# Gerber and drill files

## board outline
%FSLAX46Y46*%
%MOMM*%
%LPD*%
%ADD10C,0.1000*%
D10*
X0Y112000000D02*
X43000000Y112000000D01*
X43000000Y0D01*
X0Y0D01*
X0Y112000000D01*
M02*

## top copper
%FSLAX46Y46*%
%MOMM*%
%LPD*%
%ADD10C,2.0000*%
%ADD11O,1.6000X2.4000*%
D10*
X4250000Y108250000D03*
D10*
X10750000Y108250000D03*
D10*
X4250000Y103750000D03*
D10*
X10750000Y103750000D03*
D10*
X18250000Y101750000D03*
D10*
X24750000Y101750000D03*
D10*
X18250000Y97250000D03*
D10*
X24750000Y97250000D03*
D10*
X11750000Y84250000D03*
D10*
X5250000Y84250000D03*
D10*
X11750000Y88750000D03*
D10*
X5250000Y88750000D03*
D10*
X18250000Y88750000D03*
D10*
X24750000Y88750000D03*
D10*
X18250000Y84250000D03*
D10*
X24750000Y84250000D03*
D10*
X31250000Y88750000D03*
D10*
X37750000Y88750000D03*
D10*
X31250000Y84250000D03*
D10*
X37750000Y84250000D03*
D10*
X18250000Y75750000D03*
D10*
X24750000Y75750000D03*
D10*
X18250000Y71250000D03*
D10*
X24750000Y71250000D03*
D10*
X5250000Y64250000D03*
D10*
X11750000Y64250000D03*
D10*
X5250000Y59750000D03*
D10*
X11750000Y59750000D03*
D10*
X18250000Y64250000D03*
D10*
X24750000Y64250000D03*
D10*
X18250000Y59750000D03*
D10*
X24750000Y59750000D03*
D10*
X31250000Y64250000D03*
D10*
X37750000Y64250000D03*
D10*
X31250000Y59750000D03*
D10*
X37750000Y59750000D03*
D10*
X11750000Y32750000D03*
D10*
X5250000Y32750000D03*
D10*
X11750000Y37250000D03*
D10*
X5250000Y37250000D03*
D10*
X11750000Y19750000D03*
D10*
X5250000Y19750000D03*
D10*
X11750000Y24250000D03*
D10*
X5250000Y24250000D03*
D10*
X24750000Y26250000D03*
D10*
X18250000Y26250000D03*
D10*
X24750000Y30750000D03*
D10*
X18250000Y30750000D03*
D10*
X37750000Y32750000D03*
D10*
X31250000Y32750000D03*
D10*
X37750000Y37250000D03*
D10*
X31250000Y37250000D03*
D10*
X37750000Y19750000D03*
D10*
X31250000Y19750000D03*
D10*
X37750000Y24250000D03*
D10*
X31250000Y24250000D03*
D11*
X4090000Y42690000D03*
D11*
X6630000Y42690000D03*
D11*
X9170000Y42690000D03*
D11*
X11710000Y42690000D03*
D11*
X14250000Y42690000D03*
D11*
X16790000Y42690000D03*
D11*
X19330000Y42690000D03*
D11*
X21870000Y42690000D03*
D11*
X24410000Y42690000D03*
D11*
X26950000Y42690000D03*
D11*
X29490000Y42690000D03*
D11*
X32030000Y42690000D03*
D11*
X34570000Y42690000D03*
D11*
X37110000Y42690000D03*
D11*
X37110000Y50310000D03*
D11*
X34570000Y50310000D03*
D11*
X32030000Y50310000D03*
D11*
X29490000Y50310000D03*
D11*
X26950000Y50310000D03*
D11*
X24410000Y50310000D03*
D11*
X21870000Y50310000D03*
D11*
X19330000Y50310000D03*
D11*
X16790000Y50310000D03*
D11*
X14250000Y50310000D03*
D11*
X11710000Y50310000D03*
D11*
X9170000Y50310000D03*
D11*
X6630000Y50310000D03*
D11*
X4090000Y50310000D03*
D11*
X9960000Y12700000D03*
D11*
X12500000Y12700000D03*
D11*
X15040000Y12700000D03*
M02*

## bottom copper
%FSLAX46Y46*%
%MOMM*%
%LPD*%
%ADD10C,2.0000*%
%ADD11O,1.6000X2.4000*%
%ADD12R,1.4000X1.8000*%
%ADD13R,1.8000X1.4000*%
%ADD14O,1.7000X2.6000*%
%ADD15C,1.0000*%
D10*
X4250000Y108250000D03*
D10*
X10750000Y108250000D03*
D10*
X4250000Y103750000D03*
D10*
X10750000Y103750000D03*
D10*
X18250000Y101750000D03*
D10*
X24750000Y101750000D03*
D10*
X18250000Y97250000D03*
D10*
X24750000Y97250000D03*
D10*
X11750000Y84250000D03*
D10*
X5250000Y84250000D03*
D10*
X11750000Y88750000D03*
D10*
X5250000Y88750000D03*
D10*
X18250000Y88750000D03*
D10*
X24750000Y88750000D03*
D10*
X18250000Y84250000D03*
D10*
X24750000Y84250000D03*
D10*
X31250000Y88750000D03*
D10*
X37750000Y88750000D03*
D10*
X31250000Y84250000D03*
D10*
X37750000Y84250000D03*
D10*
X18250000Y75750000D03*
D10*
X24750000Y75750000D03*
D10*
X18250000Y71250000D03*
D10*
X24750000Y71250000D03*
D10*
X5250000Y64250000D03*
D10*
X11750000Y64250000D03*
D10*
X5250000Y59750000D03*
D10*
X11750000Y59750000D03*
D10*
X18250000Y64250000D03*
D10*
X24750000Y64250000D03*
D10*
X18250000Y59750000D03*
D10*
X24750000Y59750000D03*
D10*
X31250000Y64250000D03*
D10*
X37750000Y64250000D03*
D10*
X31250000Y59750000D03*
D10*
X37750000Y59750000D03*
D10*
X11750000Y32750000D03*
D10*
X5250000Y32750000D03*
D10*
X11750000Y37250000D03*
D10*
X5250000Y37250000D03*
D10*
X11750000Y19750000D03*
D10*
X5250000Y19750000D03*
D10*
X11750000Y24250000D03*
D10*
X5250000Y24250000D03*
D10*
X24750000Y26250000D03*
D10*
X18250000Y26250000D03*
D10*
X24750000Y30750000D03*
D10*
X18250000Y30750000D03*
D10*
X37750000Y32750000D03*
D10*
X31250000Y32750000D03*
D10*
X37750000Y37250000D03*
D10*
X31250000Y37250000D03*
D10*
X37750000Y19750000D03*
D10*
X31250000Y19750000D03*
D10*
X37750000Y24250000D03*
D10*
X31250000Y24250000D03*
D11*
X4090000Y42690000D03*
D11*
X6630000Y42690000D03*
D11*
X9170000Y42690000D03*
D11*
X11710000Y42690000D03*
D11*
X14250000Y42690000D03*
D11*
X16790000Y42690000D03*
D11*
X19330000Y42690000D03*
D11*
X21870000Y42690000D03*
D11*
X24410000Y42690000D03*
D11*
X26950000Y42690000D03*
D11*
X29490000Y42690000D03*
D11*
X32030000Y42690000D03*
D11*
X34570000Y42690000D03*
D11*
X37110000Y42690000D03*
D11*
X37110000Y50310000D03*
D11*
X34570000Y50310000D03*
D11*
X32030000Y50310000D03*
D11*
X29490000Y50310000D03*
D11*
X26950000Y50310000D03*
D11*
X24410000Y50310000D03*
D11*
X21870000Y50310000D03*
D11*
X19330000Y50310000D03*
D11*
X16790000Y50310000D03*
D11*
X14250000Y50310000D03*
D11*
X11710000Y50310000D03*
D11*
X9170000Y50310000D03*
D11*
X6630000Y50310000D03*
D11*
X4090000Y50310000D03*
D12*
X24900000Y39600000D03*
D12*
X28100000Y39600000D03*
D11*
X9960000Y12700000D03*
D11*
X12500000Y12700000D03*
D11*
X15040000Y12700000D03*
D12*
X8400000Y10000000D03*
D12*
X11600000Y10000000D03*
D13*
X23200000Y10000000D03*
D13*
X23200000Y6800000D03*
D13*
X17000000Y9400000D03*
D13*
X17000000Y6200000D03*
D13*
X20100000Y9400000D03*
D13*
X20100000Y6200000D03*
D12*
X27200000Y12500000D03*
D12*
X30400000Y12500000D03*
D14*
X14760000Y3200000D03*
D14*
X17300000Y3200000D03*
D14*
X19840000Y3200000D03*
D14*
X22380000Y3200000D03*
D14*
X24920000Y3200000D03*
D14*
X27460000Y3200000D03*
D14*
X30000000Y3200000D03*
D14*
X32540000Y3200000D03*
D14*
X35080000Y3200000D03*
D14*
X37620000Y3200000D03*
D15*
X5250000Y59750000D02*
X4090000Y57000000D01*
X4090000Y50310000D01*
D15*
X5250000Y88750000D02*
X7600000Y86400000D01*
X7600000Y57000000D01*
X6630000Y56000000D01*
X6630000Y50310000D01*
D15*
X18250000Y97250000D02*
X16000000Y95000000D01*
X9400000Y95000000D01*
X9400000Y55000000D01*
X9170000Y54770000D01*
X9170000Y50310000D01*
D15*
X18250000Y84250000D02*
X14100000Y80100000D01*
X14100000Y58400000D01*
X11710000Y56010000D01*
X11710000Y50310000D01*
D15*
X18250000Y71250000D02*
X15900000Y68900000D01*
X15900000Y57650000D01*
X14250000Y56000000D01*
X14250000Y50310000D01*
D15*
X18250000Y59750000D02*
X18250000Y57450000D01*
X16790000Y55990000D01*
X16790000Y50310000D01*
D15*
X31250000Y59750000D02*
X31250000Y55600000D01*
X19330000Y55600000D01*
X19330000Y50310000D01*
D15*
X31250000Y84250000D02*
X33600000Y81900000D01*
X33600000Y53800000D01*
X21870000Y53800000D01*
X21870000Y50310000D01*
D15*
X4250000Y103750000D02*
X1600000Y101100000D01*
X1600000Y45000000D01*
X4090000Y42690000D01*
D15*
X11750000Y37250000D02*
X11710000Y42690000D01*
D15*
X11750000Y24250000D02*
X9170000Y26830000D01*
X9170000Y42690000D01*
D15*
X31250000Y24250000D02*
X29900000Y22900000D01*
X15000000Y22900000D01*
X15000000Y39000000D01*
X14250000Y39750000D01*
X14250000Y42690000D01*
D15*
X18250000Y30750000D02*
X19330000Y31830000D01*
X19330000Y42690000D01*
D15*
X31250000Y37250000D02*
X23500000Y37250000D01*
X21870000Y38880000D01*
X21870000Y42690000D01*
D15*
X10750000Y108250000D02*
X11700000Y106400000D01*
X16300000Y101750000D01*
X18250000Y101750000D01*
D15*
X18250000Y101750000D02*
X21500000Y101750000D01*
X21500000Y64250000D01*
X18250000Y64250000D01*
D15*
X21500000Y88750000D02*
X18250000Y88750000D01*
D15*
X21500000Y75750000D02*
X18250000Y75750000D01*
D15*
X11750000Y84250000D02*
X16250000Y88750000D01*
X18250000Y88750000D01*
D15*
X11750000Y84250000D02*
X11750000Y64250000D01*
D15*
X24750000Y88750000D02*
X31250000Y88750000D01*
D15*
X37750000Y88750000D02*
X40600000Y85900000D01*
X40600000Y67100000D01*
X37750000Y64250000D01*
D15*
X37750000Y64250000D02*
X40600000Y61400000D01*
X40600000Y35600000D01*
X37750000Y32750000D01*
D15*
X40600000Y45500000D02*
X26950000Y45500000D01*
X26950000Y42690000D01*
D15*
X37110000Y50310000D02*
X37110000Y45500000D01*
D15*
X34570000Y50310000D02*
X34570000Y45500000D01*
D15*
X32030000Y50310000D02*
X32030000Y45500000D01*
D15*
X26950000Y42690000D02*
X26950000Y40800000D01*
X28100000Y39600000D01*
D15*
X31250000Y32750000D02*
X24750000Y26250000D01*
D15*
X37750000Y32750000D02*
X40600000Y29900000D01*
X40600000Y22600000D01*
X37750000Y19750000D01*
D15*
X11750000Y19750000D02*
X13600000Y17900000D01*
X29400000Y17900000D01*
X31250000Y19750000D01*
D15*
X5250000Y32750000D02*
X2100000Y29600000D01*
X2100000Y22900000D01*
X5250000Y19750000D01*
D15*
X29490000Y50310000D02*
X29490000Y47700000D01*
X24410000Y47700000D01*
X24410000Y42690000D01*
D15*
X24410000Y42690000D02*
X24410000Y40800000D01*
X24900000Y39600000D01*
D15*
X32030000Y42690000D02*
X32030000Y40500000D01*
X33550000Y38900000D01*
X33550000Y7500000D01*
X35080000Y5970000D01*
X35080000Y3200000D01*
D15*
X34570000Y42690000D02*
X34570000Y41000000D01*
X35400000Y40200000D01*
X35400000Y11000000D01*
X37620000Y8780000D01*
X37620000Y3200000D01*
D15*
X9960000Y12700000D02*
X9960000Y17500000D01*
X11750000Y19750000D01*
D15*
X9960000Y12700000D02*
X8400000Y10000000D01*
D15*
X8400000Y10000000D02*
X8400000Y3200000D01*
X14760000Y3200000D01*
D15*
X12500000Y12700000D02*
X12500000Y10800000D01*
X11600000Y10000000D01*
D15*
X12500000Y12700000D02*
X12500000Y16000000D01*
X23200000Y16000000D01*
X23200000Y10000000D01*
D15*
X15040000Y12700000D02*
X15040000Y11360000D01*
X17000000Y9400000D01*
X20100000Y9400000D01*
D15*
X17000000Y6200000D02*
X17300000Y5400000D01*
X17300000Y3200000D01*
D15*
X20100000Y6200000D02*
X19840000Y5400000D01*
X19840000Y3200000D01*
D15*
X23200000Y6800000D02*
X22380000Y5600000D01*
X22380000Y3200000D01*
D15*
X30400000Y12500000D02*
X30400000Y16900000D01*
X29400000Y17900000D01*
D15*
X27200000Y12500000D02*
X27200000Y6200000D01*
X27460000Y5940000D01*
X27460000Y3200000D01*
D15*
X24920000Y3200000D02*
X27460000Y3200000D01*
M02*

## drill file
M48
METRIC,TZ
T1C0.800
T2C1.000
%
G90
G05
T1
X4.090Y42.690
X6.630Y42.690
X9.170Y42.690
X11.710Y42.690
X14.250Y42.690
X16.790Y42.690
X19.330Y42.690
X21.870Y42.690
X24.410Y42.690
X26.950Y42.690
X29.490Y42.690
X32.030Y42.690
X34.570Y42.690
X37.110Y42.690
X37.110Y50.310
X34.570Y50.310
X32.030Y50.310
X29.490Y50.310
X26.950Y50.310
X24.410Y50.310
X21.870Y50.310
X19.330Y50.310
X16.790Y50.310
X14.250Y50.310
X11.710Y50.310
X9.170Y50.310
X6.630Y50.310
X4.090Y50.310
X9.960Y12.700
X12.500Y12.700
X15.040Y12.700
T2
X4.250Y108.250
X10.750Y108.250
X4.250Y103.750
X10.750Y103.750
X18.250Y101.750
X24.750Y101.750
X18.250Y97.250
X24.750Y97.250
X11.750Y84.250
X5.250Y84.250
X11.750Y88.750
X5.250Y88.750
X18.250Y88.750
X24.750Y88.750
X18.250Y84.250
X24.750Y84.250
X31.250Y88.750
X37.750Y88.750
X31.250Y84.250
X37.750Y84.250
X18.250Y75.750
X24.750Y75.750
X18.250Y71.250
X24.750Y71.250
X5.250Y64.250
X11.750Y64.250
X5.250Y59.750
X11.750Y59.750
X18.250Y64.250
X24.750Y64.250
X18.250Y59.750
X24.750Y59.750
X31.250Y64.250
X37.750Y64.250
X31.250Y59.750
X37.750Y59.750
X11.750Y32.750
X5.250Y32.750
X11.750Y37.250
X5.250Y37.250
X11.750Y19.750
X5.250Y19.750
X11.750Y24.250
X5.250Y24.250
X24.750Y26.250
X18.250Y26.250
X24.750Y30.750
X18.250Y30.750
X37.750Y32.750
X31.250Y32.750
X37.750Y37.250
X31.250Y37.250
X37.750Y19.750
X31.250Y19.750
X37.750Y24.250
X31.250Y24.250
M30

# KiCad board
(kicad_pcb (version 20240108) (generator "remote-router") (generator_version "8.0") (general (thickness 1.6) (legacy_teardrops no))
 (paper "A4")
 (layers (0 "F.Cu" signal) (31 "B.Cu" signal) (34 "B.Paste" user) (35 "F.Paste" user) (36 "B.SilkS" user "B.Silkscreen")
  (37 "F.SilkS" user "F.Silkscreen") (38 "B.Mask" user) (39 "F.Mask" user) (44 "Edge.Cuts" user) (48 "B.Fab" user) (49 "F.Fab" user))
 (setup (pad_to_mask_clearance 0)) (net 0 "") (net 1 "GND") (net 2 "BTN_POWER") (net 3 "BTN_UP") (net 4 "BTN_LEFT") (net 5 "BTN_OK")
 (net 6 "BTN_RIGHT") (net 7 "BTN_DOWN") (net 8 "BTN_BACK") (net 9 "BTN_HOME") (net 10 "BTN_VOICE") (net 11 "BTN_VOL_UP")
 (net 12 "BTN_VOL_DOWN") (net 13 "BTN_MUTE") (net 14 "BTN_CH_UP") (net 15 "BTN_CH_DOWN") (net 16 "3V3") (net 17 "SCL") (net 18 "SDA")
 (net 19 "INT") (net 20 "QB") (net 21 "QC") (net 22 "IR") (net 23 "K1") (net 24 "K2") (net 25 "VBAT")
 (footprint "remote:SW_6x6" (layer "F.Cu") (at 7.5000 6.0000)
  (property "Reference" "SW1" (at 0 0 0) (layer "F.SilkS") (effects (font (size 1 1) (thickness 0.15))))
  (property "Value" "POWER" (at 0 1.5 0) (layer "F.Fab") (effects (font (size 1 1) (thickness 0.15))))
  (pad "1" thru_hole circle (at -3.25 -2.25) (size 2.0 2.0) (drill 1.0) (layers "*.Cu" "*.Mask") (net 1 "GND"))
  (pad "2" thru_hole circle (at 3.25 -2.25) (size 2.0 2.0) (drill 1.0) (layers "*.Cu" "*.Mask") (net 1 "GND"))
  (pad "3" thru_hole circle (at -3.25 2.25) (size 2.0 2.0) (drill 1.0) (layers "*.Cu" "*.Mask") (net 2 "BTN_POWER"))
  (pad "4" thru_hole circle (at 3.25 2.25) (size 2.0 2.0) (drill 1.0) (layers "*.Cu" "*.Mask") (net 2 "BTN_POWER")))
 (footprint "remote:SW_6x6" (layer "F.Cu") (at 21.5000 12.5000)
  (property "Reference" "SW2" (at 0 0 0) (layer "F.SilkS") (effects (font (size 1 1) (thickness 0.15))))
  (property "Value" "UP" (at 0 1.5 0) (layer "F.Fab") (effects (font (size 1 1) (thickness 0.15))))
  (pad "1" thru_hole circle (at -3.25 -2.25) (size 2.0 2.0) (drill 1.0) (layers "*.Cu" "*.Mask") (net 1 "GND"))
  (pad "2" thru_hole circle (at 3.25 -2.25) (size 2.0 2.0) (drill 1.0) (layers "*.Cu" "*.Mask") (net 1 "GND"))
  (pad "3" thru_hole circle (at -3.25 2.25) (size 2.0 2.0) (drill 1.0) (layers "*.Cu" "*.Mask") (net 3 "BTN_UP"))
  (pad "4" thru_hole circle (at 3.25 2.25) (size 2.0 2.0) (drill 1.0) (layers "*.Cu" "*.Mask") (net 3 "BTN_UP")))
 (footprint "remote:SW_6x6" (layer "F.Cu") (at 8.5000 25.5000)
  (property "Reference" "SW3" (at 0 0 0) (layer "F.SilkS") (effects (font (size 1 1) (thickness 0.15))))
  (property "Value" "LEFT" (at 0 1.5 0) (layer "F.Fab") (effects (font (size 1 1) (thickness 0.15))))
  (pad "1" thru_hole circle (at 3.25 2.25) (size 2.0 2.0) (drill 1.0) (layers "*.Cu" "*.Mask") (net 1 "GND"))
  (pad "2" thru_hole circle (at -3.25 2.25) (size 2.0 2.0) (drill 1.0) (layers "*.Cu" "*.Mask") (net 1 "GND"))
  (pad "3" thru_hole circle (at 3.25 -2.25) (size 2.0 2.0) (drill 1.0) (layers "*.Cu" "*.Mask") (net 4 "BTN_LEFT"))
  (pad "4" thru_hole circle (at -3.25 -2.25) (size 2.0 2.0) (drill 1.0) (layers "*.Cu" "*.Mask") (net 4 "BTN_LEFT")))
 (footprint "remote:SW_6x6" (layer "F.Cu") (at 21.5000 25.5000)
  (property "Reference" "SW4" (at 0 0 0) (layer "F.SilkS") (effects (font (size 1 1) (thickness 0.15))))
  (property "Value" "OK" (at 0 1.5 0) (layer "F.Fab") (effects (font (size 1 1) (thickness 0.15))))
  (pad "1" thru_hole circle (at -3.25 -2.25) (size 2.0 2.0) (drill 1.0) (layers "*.Cu" "*.Mask") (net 1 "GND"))
  (pad "2" thru_hole circle (at 3.25 -2.25) (size 2.0 2.0) (drill 1.0) (layers "*.Cu" "*.Mask") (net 1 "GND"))
  (pad "3" thru_hole circle (at -3.25 2.25) (size 2.0 2.0) (drill 1.0) (layers "*.Cu" "*.Mask") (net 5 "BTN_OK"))
  (pad "4" thru_hole circle (at 3.25 2.25) (size 2.0 2.0) (drill 1.0) (layers "*.Cu" "*.Mask") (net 5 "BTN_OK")))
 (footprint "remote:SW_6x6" (layer "F.Cu") (at 34.5000 25.5000)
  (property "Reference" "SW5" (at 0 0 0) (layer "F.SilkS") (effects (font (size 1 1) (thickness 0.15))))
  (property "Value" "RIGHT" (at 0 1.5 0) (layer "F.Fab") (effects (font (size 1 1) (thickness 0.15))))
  (pad "1" thru_hole circle (at -3.25 -2.25) (size 2.0 2.0) (drill 1.0) (layers "*.Cu" "*.Mask") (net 1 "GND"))
  (pad "2" thru_hole circle (at 3.25 -2.25) (size 2.0 2.0) (drill 1.0) (layers "*.Cu" "*.Mask") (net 1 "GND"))
  (pad "3" thru_hole circle (at -3.25 2.25) (size 2.0 2.0) (drill 1.0) (layers "*.Cu" "*.Mask") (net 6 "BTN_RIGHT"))
  (pad "4" thru_hole circle (at 3.25 2.25) (size 2.0 2.0) (drill 1.0) (layers "*.Cu" "*.Mask") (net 6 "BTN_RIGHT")))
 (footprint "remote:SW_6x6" (layer "F.Cu") (at 21.5000 38.5000)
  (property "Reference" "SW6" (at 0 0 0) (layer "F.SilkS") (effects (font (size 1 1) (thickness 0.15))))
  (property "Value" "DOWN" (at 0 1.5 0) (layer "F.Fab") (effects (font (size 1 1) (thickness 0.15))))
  (pad "1" thru_hole circle (at -3.25 -2.25) (size 2.0 2.0) (drill 1.0) (layers "*.Cu" "*.Mask") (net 1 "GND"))
  (pad "2" thru_hole circle (at 3.25 -2.25) (size 2.0 2.0) (drill 1.0) (layers "*.Cu" "*.Mask") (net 1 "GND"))
  (pad "3" thru_hole circle (at -3.25 2.25) (size 2.0 2.0) (drill 1.0) (layers "*.Cu" "*.Mask") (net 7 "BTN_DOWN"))
  (pad "4" thru_hole circle (at 3.25 2.25) (size 2.0 2.0) (drill 1.0) (layers "*.Cu" "*.Mask") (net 7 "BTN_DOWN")))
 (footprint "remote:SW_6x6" (layer "F.Cu") (at 8.5000 50.0000)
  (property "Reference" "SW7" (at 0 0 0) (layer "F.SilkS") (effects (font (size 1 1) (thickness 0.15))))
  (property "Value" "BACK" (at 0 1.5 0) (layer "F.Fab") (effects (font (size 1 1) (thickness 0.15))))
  (pad "1" thru_hole circle (at -3.25 -2.25) (size 2.0 2.0) (drill 1.0) (layers "*.Cu" "*.Mask") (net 1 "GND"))
  (pad "2" thru_hole circle (at 3.25 -2.25) (size 2.0 2.0) (drill 1.0) (layers "*.Cu" "*.Mask") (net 1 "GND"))
  (pad "3" thru_hole circle (at -3.25 2.25) (size 2.0 2.0) (drill 1.0) (layers "*.Cu" "*.Mask") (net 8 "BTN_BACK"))
  (pad "4" thru_hole circle (at 3.25 2.25) (size 2.0 2.0) (drill 1.0) (layers "*.Cu" "*.Mask") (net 8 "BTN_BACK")))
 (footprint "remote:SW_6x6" (layer "F.Cu") (at 21.5000 50.0000)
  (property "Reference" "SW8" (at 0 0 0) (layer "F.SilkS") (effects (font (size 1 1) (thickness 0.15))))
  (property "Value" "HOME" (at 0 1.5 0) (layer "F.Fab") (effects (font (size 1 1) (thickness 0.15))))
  (pad "1" thru_hole circle (at -3.25 -2.25) (size 2.0 2.0) (drill 1.0) (layers "*.Cu" "*.Mask") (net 1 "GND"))
  (pad "2" thru_hole circle (at 3.25 -2.25) (size 2.0 2.0) (drill 1.0) (layers "*.Cu" "*.Mask") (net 1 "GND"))
  (pad "3" thru_hole circle (at -3.25 2.25) (size 2.0 2.0) (drill 1.0) (layers "*.Cu" "*.Mask") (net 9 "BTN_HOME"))
  (pad "4" thru_hole circle (at 3.25 2.25) (size 2.0 2.0) (drill 1.0) (layers "*.Cu" "*.Mask") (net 9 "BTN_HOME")))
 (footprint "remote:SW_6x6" (layer "F.Cu") (at 34.5000 50.0000)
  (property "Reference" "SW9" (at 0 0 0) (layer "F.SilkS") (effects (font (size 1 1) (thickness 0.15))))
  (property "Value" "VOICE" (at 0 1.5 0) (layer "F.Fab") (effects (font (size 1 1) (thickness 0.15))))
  (pad "1" thru_hole circle (at -3.25 -2.25) (size 2.0 2.0) (drill 1.0) (layers "*.Cu" "*.Mask") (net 1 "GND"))
  (pad "2" thru_hole circle (at 3.25 -2.25) (size 2.0 2.0) (drill 1.0) (layers "*.Cu" "*.Mask") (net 1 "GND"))
  (pad "3" thru_hole circle (at -3.25 2.25) (size 2.0 2.0) (drill 1.0) (layers "*.Cu" "*.Mask") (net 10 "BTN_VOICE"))
  (pad "4" thru_hole circle (at 3.25 2.25) (size 2.0 2.0) (drill 1.0) (layers "*.Cu" "*.Mask") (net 10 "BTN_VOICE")))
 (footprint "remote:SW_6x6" (layer "F.Cu") (at 8.5000 77.0000)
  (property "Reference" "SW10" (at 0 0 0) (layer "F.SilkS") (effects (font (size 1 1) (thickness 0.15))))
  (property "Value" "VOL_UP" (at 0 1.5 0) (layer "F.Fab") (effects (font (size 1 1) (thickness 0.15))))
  (pad "1" thru_hole circle (at 3.25 2.25) (size 2.0 2.0) (drill 1.0) (layers "*.Cu" "*.Mask") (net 1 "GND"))
  (pad "2" thru_hole circle (at -3.25 2.25) (size 2.0 2.0) (drill 1.0) (layers "*.Cu" "*.Mask") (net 1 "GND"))
  (pad "3" thru_hole circle (at 3.25 -2.25) (size 2.0 2.0) (drill 1.0) (layers "*.Cu" "*.Mask") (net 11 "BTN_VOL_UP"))
  (pad "4" thru_hole circle (at -3.25 -2.25) (size 2.0 2.0) (drill 1.0) (layers "*.Cu" "*.Mask") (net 11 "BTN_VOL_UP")))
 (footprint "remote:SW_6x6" (layer "F.Cu") (at 8.5000 90.0000)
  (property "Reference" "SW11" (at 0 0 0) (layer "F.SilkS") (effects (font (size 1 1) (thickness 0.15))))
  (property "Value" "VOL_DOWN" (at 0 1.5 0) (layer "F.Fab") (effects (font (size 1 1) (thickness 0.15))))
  (pad "1" thru_hole circle (at 3.25 2.25) (size 2.0 2.0) (drill 1.0) (layers "*.Cu" "*.Mask") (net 1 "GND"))
  (pad "2" thru_hole circle (at -3.25 2.25) (size 2.0 2.0) (drill 1.0) (layers "*.Cu" "*.Mask") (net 1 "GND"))
  (pad "3" thru_hole circle (at 3.25 -2.25) (size 2.0 2.0) (drill 1.0) (layers "*.Cu" "*.Mask") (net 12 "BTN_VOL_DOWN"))
  (pad "4" thru_hole circle (at -3.25 -2.25) (size 2.0 2.0) (drill 1.0) (layers "*.Cu" "*.Mask") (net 12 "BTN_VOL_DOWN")))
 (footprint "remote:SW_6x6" (layer "F.Cu") (at 21.5000 83.5000)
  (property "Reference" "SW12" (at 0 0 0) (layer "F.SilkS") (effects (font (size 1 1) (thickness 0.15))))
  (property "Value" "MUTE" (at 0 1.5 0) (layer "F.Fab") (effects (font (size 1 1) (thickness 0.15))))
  (pad "1" thru_hole circle (at 3.25 2.25) (size 2.0 2.0) (drill 1.0) (layers "*.Cu" "*.Mask") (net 1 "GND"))
  (pad "2" thru_hole circle (at -3.25 2.25) (size 2.0 2.0) (drill 1.0) (layers "*.Cu" "*.Mask") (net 1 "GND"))
  (pad "3" thru_hole circle (at 3.25 -2.25) (size 2.0 2.0) (drill 1.0) (layers "*.Cu" "*.Mask") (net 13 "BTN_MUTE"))
  (pad "4" thru_hole circle (at -3.25 -2.25) (size 2.0 2.0) (drill 1.0) (layers "*.Cu" "*.Mask") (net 13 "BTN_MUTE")))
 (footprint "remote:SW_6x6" (layer "F.Cu") (at 34.5000 77.0000)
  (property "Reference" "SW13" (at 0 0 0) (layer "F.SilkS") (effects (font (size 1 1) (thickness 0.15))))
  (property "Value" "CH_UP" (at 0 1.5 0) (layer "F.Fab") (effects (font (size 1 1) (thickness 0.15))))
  (pad "1" thru_hole circle (at 3.25 2.25) (size 2.0 2.0) (drill 1.0) (layers "*.Cu" "*.Mask") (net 1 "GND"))
  (pad "2" thru_hole circle (at -3.25 2.25) (size 2.0 2.0) (drill 1.0) (layers "*.Cu" "*.Mask") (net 1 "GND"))
  (pad "3" thru_hole circle (at 3.25 -2.25) (size 2.0 2.0) (drill 1.0) (layers "*.Cu" "*.Mask") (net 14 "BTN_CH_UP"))
  (pad "4" thru_hole circle (at -3.25 -2.25) (size 2.0 2.0) (drill 1.0) (layers "*.Cu" "*.Mask") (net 14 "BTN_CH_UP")))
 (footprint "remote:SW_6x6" (layer "F.Cu") (at 34.5000 90.0000)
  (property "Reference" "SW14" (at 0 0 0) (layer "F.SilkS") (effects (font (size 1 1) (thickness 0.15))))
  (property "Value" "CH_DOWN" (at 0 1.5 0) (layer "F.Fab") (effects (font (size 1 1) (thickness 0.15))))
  (pad "1" thru_hole circle (at 3.25 2.25) (size 2.0 2.0) (drill 1.0) (layers "*.Cu" "*.Mask") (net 1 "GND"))
  (pad "2" thru_hole circle (at -3.25 2.25) (size 2.0 2.0) (drill 1.0) (layers "*.Cu" "*.Mask") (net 1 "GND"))
  (pad "3" thru_hole circle (at 3.25 -2.25) (size 2.0 2.0) (drill 1.0) (layers "*.Cu" "*.Mask") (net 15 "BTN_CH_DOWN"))
  (pad "4" thru_hole circle (at -3.25 -2.25) (size 2.0 2.0) (drill 1.0) (layers "*.Cu" "*.Mask") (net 15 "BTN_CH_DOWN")))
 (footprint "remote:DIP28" (layer "F.Cu") (at 20.6000 65.5000)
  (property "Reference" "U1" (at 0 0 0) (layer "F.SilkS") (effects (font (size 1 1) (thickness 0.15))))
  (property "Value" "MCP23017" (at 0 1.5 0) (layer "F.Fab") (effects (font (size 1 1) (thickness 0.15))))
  (pad "1" thru_hole oval (at -16.51 3.81) (size 1.6 2.4) (drill 0.8) (layers "*.Cu" "*.Mask") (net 2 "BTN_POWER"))
  (pad "2" thru_hole oval (at -13.97 3.81) (size 1.6 2.4) (drill 0.8) (layers "*.Cu" "*.Mask"))
  (pad "3" thru_hole oval (at -11.43 3.81) (size 1.6 2.4) (drill 0.8) (layers "*.Cu" "*.Mask") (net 12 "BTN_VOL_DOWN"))
  (pad "4" thru_hole oval (at -8.89 3.81) (size 1.6 2.4) (drill 0.8) (layers "*.Cu" "*.Mask") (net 11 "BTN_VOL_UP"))
  (pad "5" thru_hole oval (at -6.35 3.81) (size 1.6 2.4) (drill 0.8) (layers "*.Cu" "*.Mask") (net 15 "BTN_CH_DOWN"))
  (pad "6" thru_hole oval (at -3.81 3.81) (size 1.6 2.4) (drill 0.8) (layers "*.Cu" "*.Mask"))
  (pad "7" thru_hole oval (at -1.27 3.81) (size 1.6 2.4) (drill 0.8) (layers "*.Cu" "*.Mask") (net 13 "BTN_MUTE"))
  (pad "8" thru_hole oval (at 1.27 3.81) (size 1.6 2.4) (drill 0.8) (layers "*.Cu" "*.Mask") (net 14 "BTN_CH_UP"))
  (pad "9" thru_hole oval (at 3.81 3.81) (size 1.6 2.4) (drill 0.8) (layers "*.Cu" "*.Mask") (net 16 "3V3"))
  (pad "10" thru_hole oval (at 6.35 3.81) (size 1.6 2.4) (drill 0.8) (layers "*.Cu" "*.Mask") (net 1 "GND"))
  (pad "11" thru_hole oval (at 8.89 3.81) (size 1.6 2.4) (drill 0.8) (layers "*.Cu" "*.Mask"))
  (pad "12" thru_hole oval (at 11.43 3.81) (size 1.6 2.4) (drill 0.8) (layers "*.Cu" "*.Mask") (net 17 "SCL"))
  (pad "13" thru_hole oval (at 13.97 3.81) (size 1.6 2.4) (drill 0.8) (layers "*.Cu" "*.Mask") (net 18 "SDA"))
  (pad "14" thru_hole oval (at 16.51 3.81) (size 1.6 2.4) (drill 0.8) (layers "*.Cu" "*.Mask"))
  (pad "15" thru_hole oval (at 16.51 -3.81) (size 1.6 2.4) (drill 0.8) (layers "*.Cu" "*.Mask") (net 1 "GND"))
  (pad "16" thru_hole oval (at 13.97 -3.81) (size 1.6 2.4) (drill 0.8) (layers "*.Cu" "*.Mask") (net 1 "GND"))
  (pad "17" thru_hole oval (at 11.43 -3.81) (size 1.6 2.4) (drill 0.8) (layers "*.Cu" "*.Mask") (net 1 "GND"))
  (pad "18" thru_hole oval (at 8.89 -3.81) (size 1.6 2.4) (drill 0.8) (layers "*.Cu" "*.Mask") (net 16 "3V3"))
  (pad "19" thru_hole oval (at 6.35 -3.81) (size 1.6 2.4) (drill 0.8) (layers "*.Cu" "*.Mask"))
  (pad "20" thru_hole oval (at 3.81 -3.81) (size 1.6 2.4) (drill 0.8) (layers "*.Cu" "*.Mask") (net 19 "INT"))
  (pad "21" thru_hole oval (at 1.27 -3.81) (size 1.6 2.4) (drill 0.8) (layers "*.Cu" "*.Mask") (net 6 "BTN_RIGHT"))
  (pad "22" thru_hole oval (at -1.27 -3.81) (size 1.6 2.4) (drill 0.8) (layers "*.Cu" "*.Mask") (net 10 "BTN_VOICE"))
  (pad "23" thru_hole oval (at -3.81 -3.81) (size 1.6 2.4) (drill 0.8) (layers "*.Cu" "*.Mask") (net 9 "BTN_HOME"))
  (pad "24" thru_hole oval (at -6.35 -3.81) (size 1.6 2.4) (drill 0.8) (layers "*.Cu" "*.Mask") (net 7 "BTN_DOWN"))
  (pad "25" thru_hole oval (at -8.89 -3.81) (size 1.6 2.4) (drill 0.8) (layers "*.Cu" "*.Mask") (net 5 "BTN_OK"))
  (pad "26" thru_hole oval (at -11.43 -3.81) (size 1.6 2.4) (drill 0.8) (layers "*.Cu" "*.Mask") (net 3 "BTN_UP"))
  (pad "27" thru_hole oval (at -13.97 -3.81) (size 1.6 2.4) (drill 0.8) (layers "*.Cu" "*.Mask") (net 4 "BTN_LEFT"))
  (pad "28" thru_hole oval (at -16.51 -3.81) (size 1.6 2.4) (drill 0.8) (layers "*.Cu" "*.Mask") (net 8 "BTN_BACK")))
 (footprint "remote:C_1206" (layer "F.Cu") (at 26.5000 72.4000)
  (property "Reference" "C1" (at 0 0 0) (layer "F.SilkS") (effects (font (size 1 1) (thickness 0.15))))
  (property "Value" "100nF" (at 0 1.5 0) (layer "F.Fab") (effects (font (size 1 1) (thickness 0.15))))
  (pad "1" smd rect (at -1.6 0.0) (size 1.4 1.8) (layers "B.Cu" "B.Mask") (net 16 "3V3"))
  (pad "2" smd rect (at 1.6 0.0) (size 1.4 1.8) (layers "B.Cu" "B.Mask") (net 1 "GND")))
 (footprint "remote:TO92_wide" (layer "F.Cu") (at 12.5000 99.3000)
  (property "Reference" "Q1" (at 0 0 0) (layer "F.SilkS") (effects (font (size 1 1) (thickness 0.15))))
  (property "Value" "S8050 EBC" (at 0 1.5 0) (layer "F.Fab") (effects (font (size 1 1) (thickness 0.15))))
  (pad "E" thru_hole oval (at -2.54 0.0) (size 1.6 2.4) (drill 0.8) (layers "*.Cu" "*.Mask") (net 1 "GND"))
  (pad "B" thru_hole oval (at 0.0 0.0) (size 1.6 2.4) (drill 0.8) (layers "*.Cu" "*.Mask") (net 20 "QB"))
  (pad "C" thru_hole oval (at 2.54 0.0) (size 1.6 2.4) (drill 0.8) (layers "*.Cu" "*.Mask") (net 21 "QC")))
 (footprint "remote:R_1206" (layer "F.Cu") (at 10.0000 102.0000)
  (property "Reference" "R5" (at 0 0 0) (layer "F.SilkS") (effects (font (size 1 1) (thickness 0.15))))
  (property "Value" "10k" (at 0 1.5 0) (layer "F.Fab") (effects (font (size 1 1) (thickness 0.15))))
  (pad "1" smd rect (at -1.6 0.0) (size 1.4 1.8) (layers "B.Cu" "B.Mask") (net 1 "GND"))
  (pad "2" smd rect (at 1.6 0.0) (size 1.4 1.8) (layers "B.Cu" "B.Mask") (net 20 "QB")))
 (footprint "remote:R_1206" (layer "F.Cu") (at 23.2000 103.6000)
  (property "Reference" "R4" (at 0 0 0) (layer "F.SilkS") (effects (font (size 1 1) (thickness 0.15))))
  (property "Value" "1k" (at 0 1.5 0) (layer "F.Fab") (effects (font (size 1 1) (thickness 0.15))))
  (pad "1" smd rect (at 0.0 -1.6) (size 1.8 1.4) (layers "B.Cu" "B.Mask") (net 20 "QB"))
  (pad "2" smd rect (at 0.0 1.6) (size 1.8 1.4) (layers "B.Cu" "B.Mask") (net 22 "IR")))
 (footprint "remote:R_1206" (layer "F.Cu") (at 17.0000 104.2000)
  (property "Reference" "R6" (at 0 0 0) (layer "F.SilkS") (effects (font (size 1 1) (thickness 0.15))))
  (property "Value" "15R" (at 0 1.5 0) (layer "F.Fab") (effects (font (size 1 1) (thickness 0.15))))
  (pad "1" smd rect (at 0.0 -1.6) (size 1.8 1.4) (layers "B.Cu" "B.Mask") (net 21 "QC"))
  (pad "2" smd rect (at 0.0 1.6) (size 1.8 1.4) (layers "B.Cu" "B.Mask") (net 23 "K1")))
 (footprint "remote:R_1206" (layer "F.Cu") (at 20.1000 104.2000)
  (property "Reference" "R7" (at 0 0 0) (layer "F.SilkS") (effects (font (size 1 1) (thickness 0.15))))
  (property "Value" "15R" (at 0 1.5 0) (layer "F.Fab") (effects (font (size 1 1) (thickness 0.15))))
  (pad "1" smd rect (at 0.0 -1.6) (size 1.8 1.4) (layers "B.Cu" "B.Mask") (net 21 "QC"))
  (pad "2" smd rect (at 0.0 1.6) (size 1.8 1.4) (layers "B.Cu" "B.Mask") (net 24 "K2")))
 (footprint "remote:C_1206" (layer "F.Cu") (at 28.8000 99.5000)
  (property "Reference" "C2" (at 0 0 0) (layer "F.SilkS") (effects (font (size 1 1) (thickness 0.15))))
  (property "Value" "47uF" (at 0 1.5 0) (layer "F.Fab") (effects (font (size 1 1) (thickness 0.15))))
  (pad "1" smd rect (at -1.6 0.0) (size 1.4 1.8) (layers "B.Cu" "B.Mask") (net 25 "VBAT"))
  (pad "2" smd rect (at 1.6 0.0) (size 1.4 1.8) (layers "B.Cu" "B.Mask") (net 1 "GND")))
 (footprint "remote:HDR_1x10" (layer "F.Cu") (at 26.1900 108.8000)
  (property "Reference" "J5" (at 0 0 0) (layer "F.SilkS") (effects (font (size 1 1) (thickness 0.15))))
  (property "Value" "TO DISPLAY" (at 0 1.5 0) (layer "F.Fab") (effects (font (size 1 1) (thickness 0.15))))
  (pad "1" smd oval (at -11.43 0.0) (size 1.7 2.6) (layers "B.Cu" "B.Mask") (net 1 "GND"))
  (pad "2" smd oval (at -8.89 0.0) (size 1.7 2.6) (layers "B.Cu" "B.Mask") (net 23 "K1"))
  (pad "3" smd oval (at -6.35 0.0) (size 1.7 2.6) (layers "B.Cu" "B.Mask") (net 24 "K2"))
  (pad "4" smd oval (at -3.81 0.0) (size 1.7 2.6) (layers "B.Cu" "B.Mask") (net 22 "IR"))
  (pad "5" smd oval (at -1.27 0.0) (size 1.7 2.6) (layers "B.Cu" "B.Mask") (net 25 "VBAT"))
  (pad "6" smd oval (at 1.27 0.0) (size 1.7 2.6) (layers "B.Cu" "B.Mask") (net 25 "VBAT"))
  (pad "7" smd oval (at 3.81 0.0) (size 1.7 2.6) (layers "B.Cu" "B.Mask") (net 16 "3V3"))
  (pad "8" smd oval (at 6.35 0.0) (size 1.7 2.6) (layers "B.Cu" "B.Mask") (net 19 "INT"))
  (pad "9" smd oval (at 8.89 0.0) (size 1.7 2.6) (layers "B.Cu" "B.Mask") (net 17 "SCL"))
  (pad "10" smd oval (at 11.43 0.0) (size 1.7 2.6) (layers "B.Cu" "B.Mask") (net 18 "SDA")))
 (segment (start 5.2500 52.2500) (end 4.0900 55.0000) (width 1.0) (layer "B.Cu") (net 8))
 (segment (start 4.0900 55.0000) (end 4.0900 61.6900) (width 1.0) (layer "B.Cu") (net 8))
 (segment (start 5.2500 23.2500) (end 7.6000 25.6000) (width 1.0) (layer "B.Cu") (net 4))
 (segment (start 7.6000 25.6000) (end 7.6000 55.0000) (width 1.0) (layer "B.Cu") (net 4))
 (segment (start 7.6000 55.0000) (end 6.6300 56.0000) (width 1.0) (layer "B.Cu") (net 4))
 (segment (start 6.6300 56.0000) (end 6.6300 61.6900) (width 1.0) (layer "B.Cu") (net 4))
 (segment (start 18.2500 14.7500) (end 16.0000 17.0000) (width 1.0) (layer "B.Cu") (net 3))
 (segment (start 16.0000 17.0000) (end 9.4000 17.0000) (width 1.0) (layer "B.Cu") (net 3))
 (segment (start 9.4000 17.0000) (end 9.4000 57.0000) (width 1.0) (layer "B.Cu") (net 3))
 (segment (start 9.4000 57.0000) (end 9.1700 57.2300) (width 1.0) (layer "B.Cu") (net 3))
 (segment (start 9.1700 57.2300) (end 9.1700 61.6900) (width 1.0) (layer "B.Cu") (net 3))
 (segment (start 18.2500 27.7500) (end 14.1000 31.9000) (width 1.0) (layer "B.Cu") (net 5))
 (segment (start 14.1000 31.9000) (end 14.1000 53.6000) (width 1.0) (layer "B.Cu") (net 5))
 (segment (start 14.1000 53.6000) (end 11.7100 55.9900) (width 1.0) (layer "B.Cu") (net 5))
 (segment (start 11.7100 55.9900) (end 11.7100 61.6900) (width 1.0) (layer "B.Cu") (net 5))
 (segment (start 18.2500 40.7500) (end 15.9000 43.1000) (width 1.0) (layer "B.Cu") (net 7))
 (segment (start 15.9000 43.1000) (end 15.9000 54.3500) (width 1.0) (layer "B.Cu") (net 7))
 (segment (start 15.9000 54.3500) (end 14.2500 56.0000) (width 1.0) (layer "B.Cu") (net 7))
 (segment (start 14.2500 56.0000) (end 14.2500 61.6900) (width 1.0) (layer "B.Cu") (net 7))
 (segment (start 18.2500 52.2500) (end 18.2500 54.5500) (width 1.0) (layer "B.Cu") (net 9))
 (segment (start 18.2500 54.5500) (end 16.7900 56.0100) (width 1.0) (layer "B.Cu") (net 9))
 (segment (start 16.7900 56.0100) (end 16.7900 61.6900) (width 1.0) (layer "B.Cu") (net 9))
 (segment (start 31.2500 52.2500) (end 31.2500 56.4000) (width 1.0) (layer "B.Cu") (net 10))
 (segment (start 31.2500 56.4000) (end 19.3300 56.4000) (width 1.0) (layer "B.Cu") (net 10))
 (segment (start 19.3300 56.4000) (end 19.3300 61.6900) (width 1.0) (layer "B.Cu") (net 10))
 (segment (start 31.2500 27.7500) (end 33.6000 30.1000) (width 1.0) (layer "B.Cu") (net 6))
 (segment (start 33.6000 30.1000) (end 33.6000 58.2000) (width 1.0) (layer "B.Cu") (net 6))
 (segment (start 33.6000 58.2000) (end 21.8700 58.2000) (width 1.0) (layer "B.Cu") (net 6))
 (segment (start 21.8700 58.2000) (end 21.8700 61.6900) (width 1.0) (layer "B.Cu") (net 6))
 (segment (start 4.2500 8.2500) (end 1.6000 10.9000) (width 1.0) (layer "B.Cu") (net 2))
 (segment (start 1.6000 10.9000) (end 1.6000 67.0000) (width 1.0) (layer "B.Cu") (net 2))
 (segment (start 1.6000 67.0000) (end 4.0900 69.3100) (width 1.0) (layer "B.Cu") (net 2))
 (segment (start 11.7500 74.7500) (end 11.7100 69.3100) (width 1.0) (layer "B.Cu") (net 11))
 (segment (start 11.7500 87.7500) (end 9.1700 85.1700) (width 1.0) (layer "B.Cu") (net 12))
 (segment (start 9.1700 85.1700) (end 9.1700 69.3100) (width 1.0) (layer "B.Cu") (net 12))
 (segment (start 31.2500 87.7500) (end 29.9000 89.1000) (width 1.0) (layer "B.Cu") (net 15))
 (segment (start 29.9000 89.1000) (end 15.0000 89.1000) (width 1.0) (layer "B.Cu") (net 15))
 (segment (start 15.0000 89.1000) (end 15.0000 73.0000) (width 1.0) (layer "B.Cu") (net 15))
 (segment (start 15.0000 73.0000) (end 14.2500 72.2500) (width 1.0) (layer "B.Cu") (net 15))
 (segment (start 14.2500 72.2500) (end 14.2500 69.3100) (width 1.0) (layer "B.Cu") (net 15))
 (segment (start 18.2500 81.2500) (end 19.3300 80.1700) (width 1.0) (layer "B.Cu") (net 13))
 (segment (start 19.3300 80.1700) (end 19.3300 69.3100) (width 1.0) (layer "B.Cu") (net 13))
 (segment (start 31.2500 74.7500) (end 23.5000 74.7500) (width 1.0) (layer "B.Cu") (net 14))
 (segment (start 23.5000 74.7500) (end 21.8700 73.1200) (width 1.0) (layer "B.Cu") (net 14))
 (segment (start 21.8700 73.1200) (end 21.8700 69.3100) (width 1.0) (layer "B.Cu") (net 14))
 (segment (start 10.7500 3.7500) (end 11.7000 5.6000) (width 1.0) (layer "B.Cu") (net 1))
 (segment (start 11.7000 5.6000) (end 16.3000 10.2500) (width 1.0) (layer "B.Cu") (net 1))
 (segment (start 16.3000 10.2500) (end 18.2500 10.2500) (width 1.0) (layer "B.Cu") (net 1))
 (segment (start 18.2500 10.2500) (end 21.5000 10.2500) (width 1.0) (layer "B.Cu") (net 1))
 (segment (start 21.5000 10.2500) (end 21.5000 47.7500) (width 1.0) (layer "B.Cu") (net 1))
 (segment (start 21.5000 47.7500) (end 18.2500 47.7500) (width 1.0) (layer "B.Cu") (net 1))
 (segment (start 21.5000 23.2500) (end 18.2500 23.2500) (width 1.0) (layer "B.Cu") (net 1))
 (segment (start 21.5000 36.2500) (end 18.2500 36.2500) (width 1.0) (layer "B.Cu") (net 1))
 (segment (start 11.7500 27.7500) (end 16.2500 23.2500) (width 1.0) (layer "B.Cu") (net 1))
 (segment (start 16.2500 23.2500) (end 18.2500 23.2500) (width 1.0) (layer "B.Cu") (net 1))
 (segment (start 11.7500 27.7500) (end 11.7500 47.7500) (width 1.0) (layer "B.Cu") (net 1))
 (segment (start 24.7500 23.2500) (end 31.2500 23.2500) (width 1.0) (layer "B.Cu") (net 1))
 (segment (start 37.7500 23.2500) (end 40.6000 26.1000) (width 1.0) (layer "B.Cu") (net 1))
 (segment (start 40.6000 26.1000) (end 40.6000 44.9000) (width 1.0) (layer "B.Cu") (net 1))
 (segment (start 40.6000 44.9000) (end 37.7500 47.7500) (width 1.0) (layer "B.Cu") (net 1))
 (segment (start 37.7500 47.7500) (end 40.6000 50.6000) (width 1.0) (layer "B.Cu") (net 1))
 (segment (start 40.6000 50.6000) (end 40.6000 76.4000) (width 1.0) (layer "B.Cu") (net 1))
 (segment (start 40.6000 76.4000) (end 37.7500 79.2500) (width 1.0) (layer "B.Cu") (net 1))
 (segment (start 40.6000 66.5000) (end 26.9500 66.5000) (width 1.0) (layer "B.Cu") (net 1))
 (segment (start 26.9500 66.5000) (end 26.9500 69.3100) (width 1.0) (layer "B.Cu") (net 1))
 (segment (start 37.1100 61.6900) (end 37.1100 66.5000) (width 1.0) (layer "B.Cu") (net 1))
 (segment (start 34.5700 61.6900) (end 34.5700 66.5000) (width 1.0) (layer "B.Cu") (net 1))
 (segment (start 32.0300 61.6900) (end 32.0300 66.5000) (width 1.0) (layer "B.Cu") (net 1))
 (segment (start 26.9500 69.3100) (end 26.9500 71.2000) (width 1.0) (layer "B.Cu") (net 1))
 (segment (start 26.9500 71.2000) (end 28.1000 72.4000) (width 1.0) (layer "B.Cu") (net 1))
 (segment (start 31.2500 79.2500) (end 24.7500 85.7500) (width 1.0) (layer "B.Cu") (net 1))
 (segment (start 37.7500 79.2500) (end 40.6000 82.1000) (width 1.0) (layer "B.Cu") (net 1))
 (segment (start 40.6000 82.1000) (end 40.6000 89.4000) (width 1.0) (layer "B.Cu") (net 1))
 (segment (start 40.6000 89.4000) (end 37.7500 92.2500) (width 1.0) (layer "B.Cu") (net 1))
 (segment (start 11.7500 92.2500) (end 13.6000 94.1000) (width 1.0) (layer "B.Cu") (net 1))
 (segment (start 13.6000 94.1000) (end 29.4000 94.1000) (width 1.0) (layer "B.Cu") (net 1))
 (segment (start 29.4000 94.1000) (end 31.2500 92.2500) (width 1.0) (layer "B.Cu") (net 1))
 (segment (start 5.2500 79.2500) (end 2.1000 82.4000) (width 1.0) (layer "B.Cu") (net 1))
 (segment (start 2.1000 82.4000) (end 2.1000 89.1000) (width 1.0) (layer "B.Cu") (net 1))
 (segment (start 2.1000 89.1000) (end 5.2500 92.2500) (width 1.0) (layer "B.Cu") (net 1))
 (segment (start 29.4900 61.6900) (end 29.4900 64.3000) (width 1.0) (layer "B.Cu") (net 16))
 (segment (start 29.4900 64.3000) (end 24.4100 64.3000) (width 1.0) (layer "B.Cu") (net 16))
 (segment (start 24.4100 64.3000) (end 24.4100 69.3100) (width 1.0) (layer "B.Cu") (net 16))
 (segment (start 24.4100 69.3100) (end 24.4100 71.2000) (width 1.0) (layer "B.Cu") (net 16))
 (segment (start 24.4100 71.2000) (end 24.9000 72.4000) (width 1.0) (layer "B.Cu") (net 16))
 (segment (start 32.0300 69.3100) (end 32.0300 71.5000) (width 1.0) (layer "B.Cu") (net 17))
 (segment (start 32.0300 71.5000) (end 33.5500 73.1000) (width 1.0) (layer "B.Cu") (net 17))
 (segment (start 33.5500 73.1000) (end 33.5500 104.5000) (width 1.0) (layer "B.Cu") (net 17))
 (segment (start 33.5500 104.5000) (end 35.0800 106.0300) (width 1.0) (layer "B.Cu") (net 17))
 (segment (start 35.0800 106.0300) (end 35.0800 108.8000) (width 1.0) (layer "B.Cu") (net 17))
 (segment (start 34.5700 69.3100) (end 34.5700 71.0000) (width 1.0) (layer "B.Cu") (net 18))
 (segment (start 34.5700 71.0000) (end 35.4000 71.8000) (width 1.0) (layer "B.Cu") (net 18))
 (segment (start 35.4000 71.8000) (end 35.4000 101.0000) (width 1.0) (layer "B.Cu") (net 18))
 (segment (start 35.4000 101.0000) (end 37.6200 103.2200) (width 1.0) (layer "B.Cu") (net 18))
 (segment (start 37.6200 103.2200) (end 37.6200 108.8000) (width 1.0) (layer "B.Cu") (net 18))
 (segment (start 9.9600 99.3000) (end 9.9600 94.5000) (width 1.0) (layer "B.Cu") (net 1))
 (segment (start 9.9600 94.5000) (end 11.7500 92.2500) (width 1.0) (layer "B.Cu") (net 1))
 (segment (start 9.9600 99.3000) (end 8.4000 102.0000) (width 1.0) (layer "B.Cu") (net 1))
 (segment (start 8.4000 102.0000) (end 8.4000 108.8000) (width 1.0) (layer "B.Cu") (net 1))
 (segment (start 8.4000 108.8000) (end 14.7600 108.8000) (width 1.0) (layer "B.Cu") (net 1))
 (segment (start 12.5000 99.3000) (end 12.5000 101.2000) (width 1.0) (layer "B.Cu") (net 20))
 (segment (start 12.5000 101.2000) (end 11.6000 102.0000) (width 1.0) (layer "B.Cu") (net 20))
 (segment (start 12.5000 99.3000) (end 12.5000 96.0000) (width 1.0) (layer "B.Cu") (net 20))
 (segment (start 12.5000 96.0000) (end 23.2000 96.0000) (width 1.0) (layer "B.Cu") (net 20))
 (segment (start 23.2000 96.0000) (end 23.2000 102.0000) (width 1.0) (layer "B.Cu") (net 20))
 (segment (start 15.0400 99.3000) (end 15.0400 100.6400) (width 1.0) (layer "B.Cu") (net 21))
 (segment (start 15.0400 100.6400) (end 17.0000 102.6000) (width 1.0) (layer "B.Cu") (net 21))
 (segment (start 17.0000 102.6000) (end 20.1000 102.6000) (width 1.0) (layer "B.Cu") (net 21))
 (segment (start 17.0000 105.8000) (end 17.3000 106.6000) (width 1.0) (layer "B.Cu") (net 23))
 (segment (start 17.3000 106.6000) (end 17.3000 108.8000) (width 1.0) (layer "B.Cu") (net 23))
 (segment (start 20.1000 105.8000) (end 19.8400 106.6000) (width 1.0) (layer "B.Cu") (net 24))
 (segment (start 19.8400 106.6000) (end 19.8400 108.8000) (width 1.0) (layer "B.Cu") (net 24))
 (segment (start 23.2000 105.2000) (end 22.3800 106.4000) (width 1.0) (layer "B.Cu") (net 22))
 (segment (start 22.3800 106.4000) (end 22.3800 108.8000) (width 1.0) (layer "B.Cu") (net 22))
 (segment (start 30.4000 99.5000) (end 30.4000 95.1000) (width 1.0) (layer "B.Cu") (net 1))
 (segment (start 30.4000 95.1000) (end 29.4000 94.1000) (width 1.0) (layer "B.Cu") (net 1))
 (segment (start 27.2000 99.5000) (end 27.2000 105.8000) (width 1.0) (layer "B.Cu") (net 25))
 (segment (start 27.2000 105.8000) (end 27.4600 106.0600) (width 1.0) (layer "B.Cu") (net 25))
 (segment (start 27.4600 106.0600) (end 27.4600 108.8000) (width 1.0) (layer "B.Cu") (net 25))
 (segment (start 24.9200 108.8000) (end 27.4600 108.8000) (width 1.0) (layer "B.Cu") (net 25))
 (gr_rect (start 0 0) (end 43.0 112.0) (stroke (width 0.1) (type solid)) (fill none) (layer "Edge.Cuts")))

